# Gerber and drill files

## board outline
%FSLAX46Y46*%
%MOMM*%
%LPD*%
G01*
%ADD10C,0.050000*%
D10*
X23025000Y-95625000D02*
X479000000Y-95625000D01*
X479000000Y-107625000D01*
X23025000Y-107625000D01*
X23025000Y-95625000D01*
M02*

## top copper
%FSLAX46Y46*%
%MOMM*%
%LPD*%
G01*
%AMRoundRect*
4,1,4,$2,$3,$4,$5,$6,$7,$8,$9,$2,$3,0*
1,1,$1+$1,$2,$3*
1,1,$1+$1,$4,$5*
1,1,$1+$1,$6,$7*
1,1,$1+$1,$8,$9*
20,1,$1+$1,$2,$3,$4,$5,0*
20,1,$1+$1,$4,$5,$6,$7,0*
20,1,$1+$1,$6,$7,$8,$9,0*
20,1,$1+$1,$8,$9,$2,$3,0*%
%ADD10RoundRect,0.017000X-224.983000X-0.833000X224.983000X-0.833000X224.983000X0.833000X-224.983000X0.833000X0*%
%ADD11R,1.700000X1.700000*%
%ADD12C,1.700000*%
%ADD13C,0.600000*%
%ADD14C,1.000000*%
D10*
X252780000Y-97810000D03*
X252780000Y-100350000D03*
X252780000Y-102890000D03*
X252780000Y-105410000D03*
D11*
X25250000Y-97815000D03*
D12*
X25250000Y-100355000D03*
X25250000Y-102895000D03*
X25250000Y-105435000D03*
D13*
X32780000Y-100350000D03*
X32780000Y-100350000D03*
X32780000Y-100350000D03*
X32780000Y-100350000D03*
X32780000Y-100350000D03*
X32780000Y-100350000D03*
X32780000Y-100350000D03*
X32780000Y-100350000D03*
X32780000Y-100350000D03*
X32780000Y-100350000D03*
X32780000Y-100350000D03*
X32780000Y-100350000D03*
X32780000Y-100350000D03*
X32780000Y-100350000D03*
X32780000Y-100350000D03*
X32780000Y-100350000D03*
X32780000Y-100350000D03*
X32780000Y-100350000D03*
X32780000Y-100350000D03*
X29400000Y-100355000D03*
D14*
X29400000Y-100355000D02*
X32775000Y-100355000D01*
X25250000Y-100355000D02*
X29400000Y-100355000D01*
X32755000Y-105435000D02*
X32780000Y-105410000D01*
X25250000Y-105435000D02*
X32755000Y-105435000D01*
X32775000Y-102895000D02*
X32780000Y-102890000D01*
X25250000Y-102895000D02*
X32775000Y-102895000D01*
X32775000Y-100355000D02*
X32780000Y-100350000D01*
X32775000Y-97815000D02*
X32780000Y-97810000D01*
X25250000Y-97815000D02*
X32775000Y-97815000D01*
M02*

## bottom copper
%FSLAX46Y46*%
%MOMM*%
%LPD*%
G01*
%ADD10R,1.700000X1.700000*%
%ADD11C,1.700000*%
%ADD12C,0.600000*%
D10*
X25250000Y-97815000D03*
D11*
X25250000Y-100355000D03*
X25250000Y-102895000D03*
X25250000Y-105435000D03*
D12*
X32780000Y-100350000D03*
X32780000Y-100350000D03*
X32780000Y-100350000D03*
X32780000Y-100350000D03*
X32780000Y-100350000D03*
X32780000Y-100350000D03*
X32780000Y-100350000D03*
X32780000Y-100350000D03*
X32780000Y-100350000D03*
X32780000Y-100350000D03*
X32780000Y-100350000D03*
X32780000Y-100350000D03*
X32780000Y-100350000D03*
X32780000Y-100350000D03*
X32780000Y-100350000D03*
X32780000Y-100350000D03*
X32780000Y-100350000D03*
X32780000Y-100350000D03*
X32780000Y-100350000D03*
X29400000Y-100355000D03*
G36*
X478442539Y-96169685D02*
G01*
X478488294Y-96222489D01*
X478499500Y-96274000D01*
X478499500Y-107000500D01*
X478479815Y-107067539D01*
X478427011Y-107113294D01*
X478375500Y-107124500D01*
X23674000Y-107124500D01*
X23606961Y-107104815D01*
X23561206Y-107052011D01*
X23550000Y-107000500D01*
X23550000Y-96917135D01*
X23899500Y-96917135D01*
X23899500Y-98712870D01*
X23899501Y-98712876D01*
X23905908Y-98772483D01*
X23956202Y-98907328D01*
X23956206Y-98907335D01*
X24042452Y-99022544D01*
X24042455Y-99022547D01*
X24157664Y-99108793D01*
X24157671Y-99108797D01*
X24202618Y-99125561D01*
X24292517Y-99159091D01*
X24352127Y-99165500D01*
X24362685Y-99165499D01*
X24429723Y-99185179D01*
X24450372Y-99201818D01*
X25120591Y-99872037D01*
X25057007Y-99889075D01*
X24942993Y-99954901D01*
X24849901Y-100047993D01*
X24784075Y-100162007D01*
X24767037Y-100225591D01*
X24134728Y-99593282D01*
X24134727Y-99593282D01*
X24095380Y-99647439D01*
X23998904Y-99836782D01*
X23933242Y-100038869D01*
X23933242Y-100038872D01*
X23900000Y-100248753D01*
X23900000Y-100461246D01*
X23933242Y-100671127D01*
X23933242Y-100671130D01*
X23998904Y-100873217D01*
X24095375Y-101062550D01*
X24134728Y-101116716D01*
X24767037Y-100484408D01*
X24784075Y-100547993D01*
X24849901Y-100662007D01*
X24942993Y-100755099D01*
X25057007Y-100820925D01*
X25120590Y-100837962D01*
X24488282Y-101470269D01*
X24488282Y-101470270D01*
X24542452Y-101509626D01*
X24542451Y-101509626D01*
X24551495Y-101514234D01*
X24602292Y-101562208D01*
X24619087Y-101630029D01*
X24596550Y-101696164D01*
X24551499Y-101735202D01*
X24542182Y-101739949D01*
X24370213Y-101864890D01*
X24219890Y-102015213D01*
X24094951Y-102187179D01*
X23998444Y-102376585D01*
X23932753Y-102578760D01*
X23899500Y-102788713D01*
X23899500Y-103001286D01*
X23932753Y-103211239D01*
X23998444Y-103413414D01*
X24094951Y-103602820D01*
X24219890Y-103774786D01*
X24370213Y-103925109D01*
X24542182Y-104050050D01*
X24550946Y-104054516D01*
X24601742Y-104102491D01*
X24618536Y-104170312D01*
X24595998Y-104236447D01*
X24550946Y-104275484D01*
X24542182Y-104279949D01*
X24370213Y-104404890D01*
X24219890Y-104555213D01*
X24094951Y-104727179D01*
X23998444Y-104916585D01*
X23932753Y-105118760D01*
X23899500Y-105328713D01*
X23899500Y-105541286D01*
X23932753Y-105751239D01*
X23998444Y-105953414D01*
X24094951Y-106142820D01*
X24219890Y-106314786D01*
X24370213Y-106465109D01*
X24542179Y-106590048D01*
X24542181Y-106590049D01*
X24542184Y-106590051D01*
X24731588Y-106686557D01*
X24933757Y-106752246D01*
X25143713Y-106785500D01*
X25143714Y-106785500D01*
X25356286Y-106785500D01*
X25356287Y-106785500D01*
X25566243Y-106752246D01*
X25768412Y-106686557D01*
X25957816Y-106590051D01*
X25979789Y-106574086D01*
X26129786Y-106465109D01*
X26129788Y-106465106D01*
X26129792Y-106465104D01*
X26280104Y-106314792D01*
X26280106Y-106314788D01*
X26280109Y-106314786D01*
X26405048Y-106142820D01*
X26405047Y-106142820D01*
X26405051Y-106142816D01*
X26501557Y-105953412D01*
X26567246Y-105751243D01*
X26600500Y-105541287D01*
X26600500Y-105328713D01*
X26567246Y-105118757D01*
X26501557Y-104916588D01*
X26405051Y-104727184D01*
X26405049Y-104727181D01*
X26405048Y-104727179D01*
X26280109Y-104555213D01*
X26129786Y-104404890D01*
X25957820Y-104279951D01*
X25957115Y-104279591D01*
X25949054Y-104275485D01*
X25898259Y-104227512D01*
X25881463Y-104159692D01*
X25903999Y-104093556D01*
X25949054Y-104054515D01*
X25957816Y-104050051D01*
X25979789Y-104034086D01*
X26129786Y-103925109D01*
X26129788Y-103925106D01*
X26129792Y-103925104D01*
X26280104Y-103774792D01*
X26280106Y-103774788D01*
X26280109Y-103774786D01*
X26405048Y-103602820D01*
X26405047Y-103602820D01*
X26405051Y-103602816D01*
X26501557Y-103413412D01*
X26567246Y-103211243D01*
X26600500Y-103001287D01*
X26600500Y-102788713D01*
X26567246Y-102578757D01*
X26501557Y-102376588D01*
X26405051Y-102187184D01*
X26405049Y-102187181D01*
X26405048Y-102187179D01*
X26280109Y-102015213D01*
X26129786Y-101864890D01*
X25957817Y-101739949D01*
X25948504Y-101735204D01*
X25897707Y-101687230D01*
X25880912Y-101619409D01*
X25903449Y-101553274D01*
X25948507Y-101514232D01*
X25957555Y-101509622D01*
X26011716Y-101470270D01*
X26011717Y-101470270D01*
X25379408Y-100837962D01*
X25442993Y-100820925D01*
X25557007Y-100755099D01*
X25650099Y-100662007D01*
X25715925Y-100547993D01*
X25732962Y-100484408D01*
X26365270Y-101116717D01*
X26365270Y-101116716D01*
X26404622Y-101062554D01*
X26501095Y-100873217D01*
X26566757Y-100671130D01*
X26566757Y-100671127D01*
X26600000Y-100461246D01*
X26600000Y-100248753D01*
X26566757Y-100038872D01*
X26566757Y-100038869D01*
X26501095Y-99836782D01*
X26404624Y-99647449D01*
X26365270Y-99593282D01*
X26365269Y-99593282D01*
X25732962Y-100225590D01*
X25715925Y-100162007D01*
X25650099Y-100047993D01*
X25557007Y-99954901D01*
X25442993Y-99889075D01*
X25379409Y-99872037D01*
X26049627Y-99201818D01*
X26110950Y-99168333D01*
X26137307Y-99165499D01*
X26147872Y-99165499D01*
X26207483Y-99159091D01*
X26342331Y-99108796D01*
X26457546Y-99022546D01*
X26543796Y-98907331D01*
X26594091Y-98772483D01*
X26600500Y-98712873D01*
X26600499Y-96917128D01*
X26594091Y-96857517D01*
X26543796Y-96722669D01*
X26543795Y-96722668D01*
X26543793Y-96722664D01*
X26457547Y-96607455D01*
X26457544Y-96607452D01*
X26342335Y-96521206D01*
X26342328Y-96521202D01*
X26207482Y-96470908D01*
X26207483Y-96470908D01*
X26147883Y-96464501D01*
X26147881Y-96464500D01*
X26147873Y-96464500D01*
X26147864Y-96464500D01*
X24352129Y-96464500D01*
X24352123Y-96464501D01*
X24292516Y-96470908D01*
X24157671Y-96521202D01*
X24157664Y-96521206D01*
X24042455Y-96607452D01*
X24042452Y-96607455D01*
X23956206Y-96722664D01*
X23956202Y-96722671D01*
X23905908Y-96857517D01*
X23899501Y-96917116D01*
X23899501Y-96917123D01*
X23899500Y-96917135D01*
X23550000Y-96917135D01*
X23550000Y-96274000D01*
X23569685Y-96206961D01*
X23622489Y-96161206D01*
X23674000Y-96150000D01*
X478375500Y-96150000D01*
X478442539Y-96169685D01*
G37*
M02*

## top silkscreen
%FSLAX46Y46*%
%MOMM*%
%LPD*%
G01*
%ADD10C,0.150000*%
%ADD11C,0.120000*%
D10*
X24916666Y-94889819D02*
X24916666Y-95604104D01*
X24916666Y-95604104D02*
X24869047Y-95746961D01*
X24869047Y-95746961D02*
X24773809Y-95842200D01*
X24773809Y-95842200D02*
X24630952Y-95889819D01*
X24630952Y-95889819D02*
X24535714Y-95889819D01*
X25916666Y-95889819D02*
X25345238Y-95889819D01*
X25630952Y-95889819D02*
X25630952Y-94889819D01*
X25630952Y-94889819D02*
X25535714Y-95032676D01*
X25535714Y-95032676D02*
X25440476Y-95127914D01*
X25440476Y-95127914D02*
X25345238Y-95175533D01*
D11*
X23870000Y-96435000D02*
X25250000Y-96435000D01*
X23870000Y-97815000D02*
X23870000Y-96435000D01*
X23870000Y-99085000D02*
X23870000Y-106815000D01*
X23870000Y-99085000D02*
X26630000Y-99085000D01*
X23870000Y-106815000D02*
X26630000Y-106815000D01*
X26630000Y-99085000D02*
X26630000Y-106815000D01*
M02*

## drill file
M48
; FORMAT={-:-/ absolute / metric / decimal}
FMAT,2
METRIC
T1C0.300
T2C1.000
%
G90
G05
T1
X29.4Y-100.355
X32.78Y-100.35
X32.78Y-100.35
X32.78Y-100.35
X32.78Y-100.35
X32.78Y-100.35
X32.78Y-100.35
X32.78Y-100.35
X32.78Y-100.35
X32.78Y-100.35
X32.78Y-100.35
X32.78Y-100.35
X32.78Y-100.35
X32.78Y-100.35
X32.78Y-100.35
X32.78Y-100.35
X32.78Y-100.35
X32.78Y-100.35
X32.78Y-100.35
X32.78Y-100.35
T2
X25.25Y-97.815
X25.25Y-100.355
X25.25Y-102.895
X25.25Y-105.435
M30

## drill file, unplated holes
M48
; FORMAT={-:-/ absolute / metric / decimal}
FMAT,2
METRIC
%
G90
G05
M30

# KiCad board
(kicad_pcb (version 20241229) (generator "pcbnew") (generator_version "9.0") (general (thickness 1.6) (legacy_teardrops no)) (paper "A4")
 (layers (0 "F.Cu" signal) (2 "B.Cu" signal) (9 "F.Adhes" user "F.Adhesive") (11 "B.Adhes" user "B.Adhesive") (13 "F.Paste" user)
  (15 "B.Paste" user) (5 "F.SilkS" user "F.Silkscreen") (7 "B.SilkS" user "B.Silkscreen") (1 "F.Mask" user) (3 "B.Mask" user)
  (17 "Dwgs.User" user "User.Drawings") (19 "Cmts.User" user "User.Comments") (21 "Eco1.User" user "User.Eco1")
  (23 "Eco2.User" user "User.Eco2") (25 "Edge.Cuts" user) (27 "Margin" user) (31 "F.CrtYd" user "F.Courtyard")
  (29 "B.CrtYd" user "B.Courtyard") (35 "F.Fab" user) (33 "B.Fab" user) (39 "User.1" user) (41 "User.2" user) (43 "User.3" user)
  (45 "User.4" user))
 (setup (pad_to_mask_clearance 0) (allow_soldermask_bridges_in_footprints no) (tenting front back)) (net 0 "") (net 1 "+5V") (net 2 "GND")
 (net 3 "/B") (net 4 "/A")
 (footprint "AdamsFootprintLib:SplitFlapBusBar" (layer "F.Cu") (at 32.78 97.81)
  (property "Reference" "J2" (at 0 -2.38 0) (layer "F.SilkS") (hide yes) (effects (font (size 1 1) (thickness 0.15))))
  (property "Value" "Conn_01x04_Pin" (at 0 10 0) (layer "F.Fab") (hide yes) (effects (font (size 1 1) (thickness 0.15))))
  (pad "1" smd roundrect (at 0 0) (size 450 1.7) (drill (offset 220 0)) (layers "F.Cu" "F.Mask" "F.Paste") (roundrect_rratio 0.01)
   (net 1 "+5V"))
  (pad "2" smd roundrect (at 0 2.54) (size 450 1.7) (drill (offset 220 0)) (layers "F.Cu" "F.Mask" "F.Paste") (roundrect_rratio 0.01)
   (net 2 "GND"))
  (pad "3" smd roundrect (at 0 5.08) (size 450 1.7) (drill (offset 220 0)) (layers "F.Cu" "F.Mask" "F.Paste") (roundrect_rratio 0.01)
   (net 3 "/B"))
  (pad "4" smd roundrect (at 0 7.6) (size 450 1.7) (drill (offset 220 0)) (layers "F.Cu" "F.Mask" "F.Paste") (roundrect_rratio 0.01)
   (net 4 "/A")))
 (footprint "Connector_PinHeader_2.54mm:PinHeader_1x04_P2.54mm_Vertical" (layer "F.Cu") (at 25.25 97.815)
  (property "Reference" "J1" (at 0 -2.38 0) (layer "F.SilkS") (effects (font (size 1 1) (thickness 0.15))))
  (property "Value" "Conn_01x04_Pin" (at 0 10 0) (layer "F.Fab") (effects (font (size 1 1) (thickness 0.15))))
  (fp_line (start -1.38 -1.38) (end 0 -1.38) (stroke (width 0.12) (type solid)) (layer "F.SilkS"))
  (fp_line (start -1.38 0) (end -1.38 -1.38) (stroke (width 0.12) (type solid)) (layer "F.SilkS"))
  (fp_line (start -1.38 1.27) (end -1.38 9) (stroke (width 0.12) (type solid)) (layer "F.SilkS"))
  (fp_line (start -1.38 1.27) (end 1.38 1.27) (stroke (width 0.12) (type solid)) (layer "F.SilkS"))
  (fp_line (start -1.38 9) (end 1.38 9) (stroke (width 0.12) (type solid)) (layer "F.SilkS"))
  (fp_line (start 1.38 1.27) (end 1.38 9) (stroke (width 0.12) (type solid)) (layer "F.SilkS"))
  (pad "1" thru_hole rect (at 0 0) (size 1.7 1.7) (drill 1) (layers "*.Cu" "*.Mask") (remove_unused_layers no) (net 1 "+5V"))
  (pad "2" thru_hole circle (at 0 2.54) (size 1.7 1.7) (drill 1) (layers "*.Cu" "*.Mask") (remove_unused_layers no) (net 2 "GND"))
  (pad "3" thru_hole circle (at 0 5.08) (size 1.7 1.7) (drill 1) (layers "*.Cu" "*.Mask") (remove_unused_layers no) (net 3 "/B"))
  (pad "4" thru_hole circle (at 0 7.62) (size 1.7 1.7) (drill 1) (layers "*.Cu" "*.Mask") (remove_unused_layers no) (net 4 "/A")))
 (gr_rect (start 23.025 95.625) (end 479 107.625) (stroke (width 0.05) (type solid)) (fill no) (layer "Edge.Cuts"))
 (segment (start 32.775 97.815) (end 32.78 97.81) (width 1) (layer "F.Cu") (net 1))
 (segment (start 25.25 97.815) (end 32.775 97.815) (width 1) (layer "F.Cu") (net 1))
 (segment (start 32.775 102.895) (end 32.78 102.89) (width 1) (layer "F.Cu") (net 3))
 (segment (start 25.25 102.895) (end 32.775 102.895) (width 1) (layer "F.Cu") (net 3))
 (segment (start 32.755 105.435) (end 32.78 105.41) (width 1) (layer "F.Cu") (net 4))
 (segment (start 25.25 105.435) (end 32.755 105.435) (width 1) (layer "F.Cu") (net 4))
 (segment (start 25.25 100.355) (end 29.4 100.355) (width 1) (layer "F.Cu") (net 2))
 (segment (start 32.775 100.355) (end 32.78 100.35) (width 1) (layer "F.Cu") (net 2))
 (segment (start 29.4 100.355) (end 32.775 100.355) (width 1) (layer "F.Cu") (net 2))
 (via (at 32.78 100.35) (size 0.6) (drill 0.3) (layers "F.Cu" "B.Cu") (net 2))
 (via (at 32.78 100.35) (size 0.6) (drill 0.3) (layers "F.Cu" "B.Cu") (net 2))
 (via (at 32.78 100.35) (size 0.6) (drill 0.3) (layers "F.Cu" "B.Cu") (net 2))
 (via (at 32.78 100.35) (size 0.6) (drill 0.3) (layers "F.Cu" "B.Cu") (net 2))
 (via (at 29.4 100.355) (size 0.6) (drill 0.3) (layers "F.Cu" "B.Cu") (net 2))
 (via (at 32.78 100.35) (size 0.6) (drill 0.3) (layers "F.Cu" "B.Cu") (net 2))
 (via (at 32.78 100.35) (size 0.6) (drill 0.3) (layers "F.Cu" "B.Cu") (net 2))
 (via (at 32.78 100.35) (size 0.6) (drill 0.3) (layers "F.Cu" "B.Cu") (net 2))
 (via (at 32.78 100.35) (size 0.6) (drill 0.3) (layers "F.Cu" "B.Cu") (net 2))
 (via (at 32.78 100.35) (size 0.6) (drill 0.3) (layers "F.Cu" "B.Cu") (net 2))
 (via (at 32.78 100.35) (size 0.6) (drill 0.3) (layers "F.Cu" "B.Cu") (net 2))
 (via (at 32.78 100.35) (size 0.6) (drill 0.3) (layers "F.Cu" "B.Cu") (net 2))
 (via (at 32.78 100.35) (size 0.6) (drill 0.3) (layers "F.Cu" "B.Cu") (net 2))
 (via (at 32.78 100.35) (size 0.6) (drill 0.3) (layers "F.Cu" "B.Cu") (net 2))
 (via (at 32.78 100.35) (size 0.6) (drill 0.3) (layers "F.Cu" "B.Cu") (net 2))
 (via (at 32.78 100.35) (size 0.6) (drill 0.3) (layers "F.Cu" "B.Cu") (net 2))
 (via (at 32.78 100.35) (size 0.6) (drill 0.3) (layers "F.Cu" "B.Cu") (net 2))
 (via (at 32.78 100.35) (size 0.6) (drill 0.3) (layers "F.Cu" "B.Cu") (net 2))
 (via (at 32.78 100.35) (size 0.6) (drill 0.3) (layers "F.Cu" "B.Cu") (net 2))
 (via (at 32.78 100.35) (size 0.6) (drill 0.3) (layers "F.Cu" "B.Cu") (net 2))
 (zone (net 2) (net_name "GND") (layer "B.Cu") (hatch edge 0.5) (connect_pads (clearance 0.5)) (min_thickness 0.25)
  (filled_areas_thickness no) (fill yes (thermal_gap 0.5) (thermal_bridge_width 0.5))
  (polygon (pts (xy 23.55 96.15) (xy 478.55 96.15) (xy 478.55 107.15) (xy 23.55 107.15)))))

